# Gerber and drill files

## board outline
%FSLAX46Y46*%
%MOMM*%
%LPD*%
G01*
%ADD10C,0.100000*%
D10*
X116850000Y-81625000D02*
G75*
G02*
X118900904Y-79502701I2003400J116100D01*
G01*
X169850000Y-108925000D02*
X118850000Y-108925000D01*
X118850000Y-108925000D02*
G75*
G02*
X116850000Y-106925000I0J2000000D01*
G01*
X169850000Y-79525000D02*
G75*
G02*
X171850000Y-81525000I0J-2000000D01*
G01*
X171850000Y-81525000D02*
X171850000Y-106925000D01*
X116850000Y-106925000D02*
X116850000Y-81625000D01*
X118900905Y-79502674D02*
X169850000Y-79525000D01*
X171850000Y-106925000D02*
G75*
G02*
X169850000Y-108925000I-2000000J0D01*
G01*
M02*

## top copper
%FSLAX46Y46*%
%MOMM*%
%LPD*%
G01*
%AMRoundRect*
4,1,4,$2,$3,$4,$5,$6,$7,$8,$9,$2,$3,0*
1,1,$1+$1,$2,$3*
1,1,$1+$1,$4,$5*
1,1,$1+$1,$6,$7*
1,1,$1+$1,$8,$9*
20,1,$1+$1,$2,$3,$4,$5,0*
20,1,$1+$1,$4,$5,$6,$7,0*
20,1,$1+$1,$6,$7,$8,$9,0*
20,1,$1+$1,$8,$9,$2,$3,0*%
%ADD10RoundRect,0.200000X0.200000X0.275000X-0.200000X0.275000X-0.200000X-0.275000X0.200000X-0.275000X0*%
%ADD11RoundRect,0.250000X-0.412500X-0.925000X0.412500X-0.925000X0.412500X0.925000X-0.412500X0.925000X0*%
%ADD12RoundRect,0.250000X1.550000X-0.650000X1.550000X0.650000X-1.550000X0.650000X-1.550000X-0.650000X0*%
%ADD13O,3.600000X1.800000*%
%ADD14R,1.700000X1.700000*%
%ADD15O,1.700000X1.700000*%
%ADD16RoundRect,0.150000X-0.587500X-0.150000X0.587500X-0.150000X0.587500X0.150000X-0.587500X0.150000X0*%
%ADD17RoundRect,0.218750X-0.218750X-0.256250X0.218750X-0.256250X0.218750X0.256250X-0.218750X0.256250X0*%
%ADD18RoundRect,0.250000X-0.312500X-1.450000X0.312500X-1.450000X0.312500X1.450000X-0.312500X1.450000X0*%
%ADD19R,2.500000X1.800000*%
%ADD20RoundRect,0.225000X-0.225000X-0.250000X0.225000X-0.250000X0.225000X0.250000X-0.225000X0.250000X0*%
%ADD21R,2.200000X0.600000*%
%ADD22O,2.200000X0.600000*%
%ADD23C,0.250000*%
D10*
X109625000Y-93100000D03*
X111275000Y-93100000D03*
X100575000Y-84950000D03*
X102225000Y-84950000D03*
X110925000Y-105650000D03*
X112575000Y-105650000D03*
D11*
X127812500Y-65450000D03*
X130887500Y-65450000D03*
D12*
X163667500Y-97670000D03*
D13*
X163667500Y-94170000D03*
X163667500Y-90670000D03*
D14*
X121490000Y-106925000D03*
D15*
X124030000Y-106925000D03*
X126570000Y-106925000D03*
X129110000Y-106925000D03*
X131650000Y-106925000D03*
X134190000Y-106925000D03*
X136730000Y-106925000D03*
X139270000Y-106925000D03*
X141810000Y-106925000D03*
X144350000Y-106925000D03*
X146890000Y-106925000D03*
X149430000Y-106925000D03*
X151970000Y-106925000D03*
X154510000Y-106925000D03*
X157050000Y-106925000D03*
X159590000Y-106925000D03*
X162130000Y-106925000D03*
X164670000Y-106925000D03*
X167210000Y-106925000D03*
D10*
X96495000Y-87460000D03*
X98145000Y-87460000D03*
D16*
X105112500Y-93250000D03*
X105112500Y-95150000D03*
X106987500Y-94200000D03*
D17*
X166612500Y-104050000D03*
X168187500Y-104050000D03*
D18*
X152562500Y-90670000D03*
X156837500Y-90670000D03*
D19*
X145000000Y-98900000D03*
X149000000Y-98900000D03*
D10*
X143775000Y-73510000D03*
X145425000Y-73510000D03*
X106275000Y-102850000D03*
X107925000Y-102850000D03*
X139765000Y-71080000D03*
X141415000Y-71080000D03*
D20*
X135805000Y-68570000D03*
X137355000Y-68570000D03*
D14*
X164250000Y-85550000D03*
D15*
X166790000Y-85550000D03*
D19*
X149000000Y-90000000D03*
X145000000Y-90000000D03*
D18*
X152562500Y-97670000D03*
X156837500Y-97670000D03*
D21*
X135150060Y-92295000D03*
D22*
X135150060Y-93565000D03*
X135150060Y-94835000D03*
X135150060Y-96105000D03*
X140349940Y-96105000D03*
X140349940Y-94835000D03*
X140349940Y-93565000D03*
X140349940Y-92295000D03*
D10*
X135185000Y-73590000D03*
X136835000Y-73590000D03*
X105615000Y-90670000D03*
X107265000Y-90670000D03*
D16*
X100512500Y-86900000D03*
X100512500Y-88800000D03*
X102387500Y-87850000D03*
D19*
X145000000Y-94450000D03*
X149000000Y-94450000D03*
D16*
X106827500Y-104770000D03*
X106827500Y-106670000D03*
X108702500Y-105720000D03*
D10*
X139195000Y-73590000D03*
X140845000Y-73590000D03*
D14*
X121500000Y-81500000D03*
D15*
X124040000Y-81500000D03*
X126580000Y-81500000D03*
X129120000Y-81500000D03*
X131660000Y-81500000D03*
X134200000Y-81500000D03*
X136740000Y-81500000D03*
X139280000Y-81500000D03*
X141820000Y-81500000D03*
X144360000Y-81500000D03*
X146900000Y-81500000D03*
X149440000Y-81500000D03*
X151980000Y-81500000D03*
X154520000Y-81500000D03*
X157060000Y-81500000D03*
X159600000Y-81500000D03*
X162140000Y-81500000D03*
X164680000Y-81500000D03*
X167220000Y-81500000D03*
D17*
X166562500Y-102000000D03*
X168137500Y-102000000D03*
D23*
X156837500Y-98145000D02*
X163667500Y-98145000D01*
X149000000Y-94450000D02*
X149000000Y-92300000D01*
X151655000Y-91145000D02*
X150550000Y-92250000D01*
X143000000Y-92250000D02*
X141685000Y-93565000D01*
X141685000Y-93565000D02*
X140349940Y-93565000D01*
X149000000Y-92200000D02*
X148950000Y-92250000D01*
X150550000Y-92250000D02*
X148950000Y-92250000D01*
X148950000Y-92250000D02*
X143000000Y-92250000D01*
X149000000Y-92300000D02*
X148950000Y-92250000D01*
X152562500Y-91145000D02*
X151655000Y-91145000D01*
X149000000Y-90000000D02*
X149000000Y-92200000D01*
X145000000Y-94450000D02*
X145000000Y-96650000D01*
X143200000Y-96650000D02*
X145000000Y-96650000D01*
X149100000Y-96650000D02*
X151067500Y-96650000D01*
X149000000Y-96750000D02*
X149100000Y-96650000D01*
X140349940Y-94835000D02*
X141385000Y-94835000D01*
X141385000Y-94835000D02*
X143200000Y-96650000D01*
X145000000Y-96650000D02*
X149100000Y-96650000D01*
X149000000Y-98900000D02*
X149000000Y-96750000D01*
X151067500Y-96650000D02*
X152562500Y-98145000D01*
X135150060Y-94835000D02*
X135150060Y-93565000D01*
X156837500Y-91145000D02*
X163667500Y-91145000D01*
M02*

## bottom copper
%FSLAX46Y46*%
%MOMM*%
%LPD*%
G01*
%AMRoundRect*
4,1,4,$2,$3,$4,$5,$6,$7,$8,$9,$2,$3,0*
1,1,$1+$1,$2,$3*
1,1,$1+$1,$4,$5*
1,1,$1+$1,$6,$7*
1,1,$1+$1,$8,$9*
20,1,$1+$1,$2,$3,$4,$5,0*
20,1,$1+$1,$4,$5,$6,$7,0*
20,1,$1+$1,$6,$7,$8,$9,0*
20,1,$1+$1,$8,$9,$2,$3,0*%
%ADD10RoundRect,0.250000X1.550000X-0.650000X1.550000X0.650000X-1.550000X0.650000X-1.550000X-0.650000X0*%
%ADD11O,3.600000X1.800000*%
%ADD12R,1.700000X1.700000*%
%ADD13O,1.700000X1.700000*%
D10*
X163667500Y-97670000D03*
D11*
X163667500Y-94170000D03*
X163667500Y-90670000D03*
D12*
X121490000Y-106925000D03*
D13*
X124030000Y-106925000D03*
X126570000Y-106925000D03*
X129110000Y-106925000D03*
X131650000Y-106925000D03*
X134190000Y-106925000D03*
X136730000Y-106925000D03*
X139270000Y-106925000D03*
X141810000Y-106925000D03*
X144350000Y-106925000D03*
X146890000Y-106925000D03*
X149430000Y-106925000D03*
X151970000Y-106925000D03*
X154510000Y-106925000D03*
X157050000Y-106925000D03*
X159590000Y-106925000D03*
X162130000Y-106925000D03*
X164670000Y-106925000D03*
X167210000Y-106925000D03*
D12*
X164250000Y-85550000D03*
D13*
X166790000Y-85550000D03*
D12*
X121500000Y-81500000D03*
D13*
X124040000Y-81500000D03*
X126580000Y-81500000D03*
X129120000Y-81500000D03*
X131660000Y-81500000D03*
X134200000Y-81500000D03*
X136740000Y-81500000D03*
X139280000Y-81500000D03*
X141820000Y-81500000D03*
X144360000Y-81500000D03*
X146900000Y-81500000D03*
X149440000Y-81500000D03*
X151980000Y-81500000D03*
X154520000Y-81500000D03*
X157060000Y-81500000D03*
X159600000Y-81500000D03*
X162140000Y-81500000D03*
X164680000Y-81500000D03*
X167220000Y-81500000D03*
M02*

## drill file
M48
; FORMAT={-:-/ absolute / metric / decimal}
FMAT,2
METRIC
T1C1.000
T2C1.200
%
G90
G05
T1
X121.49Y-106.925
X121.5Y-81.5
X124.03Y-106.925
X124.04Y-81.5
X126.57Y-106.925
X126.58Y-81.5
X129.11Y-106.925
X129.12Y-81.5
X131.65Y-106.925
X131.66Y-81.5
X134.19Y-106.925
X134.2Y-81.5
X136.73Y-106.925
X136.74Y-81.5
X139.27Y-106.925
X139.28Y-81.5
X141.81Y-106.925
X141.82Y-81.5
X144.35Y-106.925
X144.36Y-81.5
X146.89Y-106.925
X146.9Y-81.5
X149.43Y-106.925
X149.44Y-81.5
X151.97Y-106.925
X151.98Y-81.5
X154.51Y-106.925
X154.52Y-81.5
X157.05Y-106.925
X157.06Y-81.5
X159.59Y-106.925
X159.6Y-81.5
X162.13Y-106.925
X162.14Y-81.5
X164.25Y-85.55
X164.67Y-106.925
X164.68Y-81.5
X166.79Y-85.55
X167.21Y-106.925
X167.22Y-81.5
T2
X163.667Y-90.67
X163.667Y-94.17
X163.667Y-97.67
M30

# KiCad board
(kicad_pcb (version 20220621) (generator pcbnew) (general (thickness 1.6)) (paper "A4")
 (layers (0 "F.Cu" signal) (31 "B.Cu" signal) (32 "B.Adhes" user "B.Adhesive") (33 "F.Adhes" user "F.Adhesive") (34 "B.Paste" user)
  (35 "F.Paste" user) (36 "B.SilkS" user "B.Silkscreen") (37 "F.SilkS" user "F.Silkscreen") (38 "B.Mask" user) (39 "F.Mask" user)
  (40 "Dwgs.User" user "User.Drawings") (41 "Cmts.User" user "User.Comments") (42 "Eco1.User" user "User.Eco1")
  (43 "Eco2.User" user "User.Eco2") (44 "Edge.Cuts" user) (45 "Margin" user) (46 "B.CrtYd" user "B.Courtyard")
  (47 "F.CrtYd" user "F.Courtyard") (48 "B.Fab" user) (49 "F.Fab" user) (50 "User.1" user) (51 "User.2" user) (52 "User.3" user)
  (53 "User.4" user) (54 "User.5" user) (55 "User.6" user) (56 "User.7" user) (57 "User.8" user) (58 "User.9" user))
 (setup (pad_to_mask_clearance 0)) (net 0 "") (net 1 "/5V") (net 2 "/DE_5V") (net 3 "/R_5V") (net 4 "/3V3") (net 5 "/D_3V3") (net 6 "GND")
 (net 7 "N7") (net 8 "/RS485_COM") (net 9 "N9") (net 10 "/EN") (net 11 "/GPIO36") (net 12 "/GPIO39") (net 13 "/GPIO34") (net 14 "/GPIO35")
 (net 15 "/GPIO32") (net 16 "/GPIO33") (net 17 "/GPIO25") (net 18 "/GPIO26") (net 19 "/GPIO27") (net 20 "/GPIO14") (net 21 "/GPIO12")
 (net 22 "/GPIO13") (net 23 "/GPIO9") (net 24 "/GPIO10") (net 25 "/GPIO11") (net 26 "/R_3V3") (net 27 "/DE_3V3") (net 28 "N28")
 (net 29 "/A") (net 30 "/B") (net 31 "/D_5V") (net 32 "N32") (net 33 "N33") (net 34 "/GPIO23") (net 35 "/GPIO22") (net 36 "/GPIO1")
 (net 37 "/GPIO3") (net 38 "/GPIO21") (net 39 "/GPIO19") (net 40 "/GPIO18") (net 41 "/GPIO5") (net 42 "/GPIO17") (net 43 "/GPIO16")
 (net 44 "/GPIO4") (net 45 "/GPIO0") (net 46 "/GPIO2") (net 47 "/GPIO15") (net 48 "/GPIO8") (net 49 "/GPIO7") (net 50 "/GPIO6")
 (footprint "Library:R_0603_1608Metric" (layer "F.Cu") (at 110.45 93.1)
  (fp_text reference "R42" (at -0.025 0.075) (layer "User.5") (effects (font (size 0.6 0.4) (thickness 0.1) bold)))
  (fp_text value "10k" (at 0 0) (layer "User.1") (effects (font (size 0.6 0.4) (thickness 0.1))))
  (pad "1" smd roundrect (at -0.825 0 180) (size 0.8 0.95) (layers "F.Cu" "F.Paste" "F.Mask") (roundrect_rratio 0.25) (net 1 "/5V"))
  (pad "2" smd roundrect (at 0.825 0 180) (size 0.8 0.95) (layers "F.Cu" "F.Paste" "F.Mask") (roundrect_rratio 0.25) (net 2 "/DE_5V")))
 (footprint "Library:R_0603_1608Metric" (layer "F.Cu") (at 101.4 84.95)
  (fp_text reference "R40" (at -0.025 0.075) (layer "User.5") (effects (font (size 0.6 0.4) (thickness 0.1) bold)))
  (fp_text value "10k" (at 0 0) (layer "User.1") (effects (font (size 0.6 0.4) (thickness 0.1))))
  (pad "1" smd roundrect (at -0.825 0 180) (size 0.8 0.95) (layers "F.Cu" "F.Paste" "F.Mask") (roundrect_rratio 0.25) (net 1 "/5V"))
  (pad "2" smd roundrect (at 0.825 0 180) (size 0.8 0.95) (layers "F.Cu" "F.Paste" "F.Mask") (roundrect_rratio 0.25) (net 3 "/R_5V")))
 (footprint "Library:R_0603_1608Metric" (layer "F.Cu") (at 111.75 105.65)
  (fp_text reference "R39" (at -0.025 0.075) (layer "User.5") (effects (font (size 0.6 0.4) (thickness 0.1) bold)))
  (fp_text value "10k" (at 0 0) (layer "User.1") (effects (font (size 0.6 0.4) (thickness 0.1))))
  (pad "1" smd roundrect (at -0.825 0 180) (size 0.8 0.95) (layers "F.Cu" "F.Paste" "F.Mask") (roundrect_rratio 0.25) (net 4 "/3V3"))
  (pad "2" smd roundrect (at 0.825 0 180) (size 0.8 0.95) (layers "F.Cu" "F.Paste" "F.Mask") (roundrect_rratio 0.25) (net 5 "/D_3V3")))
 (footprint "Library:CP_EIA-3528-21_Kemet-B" (layer "F.Cu") (at 129.35 65.45)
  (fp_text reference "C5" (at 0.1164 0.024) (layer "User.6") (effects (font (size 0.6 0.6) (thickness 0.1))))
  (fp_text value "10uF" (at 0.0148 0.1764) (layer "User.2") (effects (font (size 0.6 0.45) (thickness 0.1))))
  (pad "1" smd roundrect (at -1.5375 0) (size 1.325 2.35) (layers "F.Cu" "F.Paste" "F.Mask") (roundrect_rratio 0.1886792453) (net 1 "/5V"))
  (pad "2" smd roundrect (at 1.5375 0) (size 1.325 2.35) (layers "F.Cu" "F.Paste" "F.Mask") (roundrect_rratio 0.1886792453) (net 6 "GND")))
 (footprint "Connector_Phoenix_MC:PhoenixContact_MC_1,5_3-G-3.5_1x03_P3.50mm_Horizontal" (layer "F.Cu") (at 163.6675 97.67 90)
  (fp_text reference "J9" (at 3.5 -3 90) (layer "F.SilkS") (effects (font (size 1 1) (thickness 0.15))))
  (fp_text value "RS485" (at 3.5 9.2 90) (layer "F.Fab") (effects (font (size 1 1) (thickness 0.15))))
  (pad "1" thru_hole roundrect (at 0 0 90) (size 1.8 3.6) (drill 1.2) (layers *.Cu *.Mask) (roundrect_rratio 0.138889) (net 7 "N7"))
  (pad "2" thru_hole oval (at 3.5 0 90) (size 1.8 3.6) (drill 1.2) (layers *.Cu *.Mask) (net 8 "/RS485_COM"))
  (pad "3" thru_hole oval (at 7 0 90) (size 1.8 3.6) (drill 1.2) (layers *.Cu *.Mask) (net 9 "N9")))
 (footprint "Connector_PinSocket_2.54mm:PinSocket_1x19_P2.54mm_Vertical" (layer "F.Cu") (at 121.49 106.925 90)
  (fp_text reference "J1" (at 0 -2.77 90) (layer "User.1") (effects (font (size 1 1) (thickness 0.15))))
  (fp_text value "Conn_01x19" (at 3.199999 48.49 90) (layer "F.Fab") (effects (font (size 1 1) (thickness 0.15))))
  (pad "1" thru_hole rect (at 0 0 90) (size 1.7 1.7) (drill 1) (layers *.Cu *.Mask) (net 4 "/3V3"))
  (pad "2" thru_hole oval (at 0 2.54 90) (size 1.7 1.7) (drill 1) (layers *.Cu *.Mask) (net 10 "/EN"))
  (pad "3" thru_hole oval (at 0 5.08 90) (size 1.7 1.7) (drill 1) (layers *.Cu *.Mask) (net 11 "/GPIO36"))
  (pad "4" thru_hole oval (at 0 7.62 90) (size 1.7 1.7) (drill 1) (layers *.Cu *.Mask) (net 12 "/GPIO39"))
  (pad "5" thru_hole oval (at 0 10.16 90) (size 1.7 1.7) (drill 1) (layers *.Cu *.Mask) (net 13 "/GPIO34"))
  (pad "6" thru_hole oval (at 0 12.7 90) (size 1.7 1.7) (drill 1) (layers *.Cu *.Mask) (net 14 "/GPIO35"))
  (pad "7" thru_hole oval (at 0 15.24 90) (size 1.7 1.7) (drill 1) (layers *.Cu *.Mask) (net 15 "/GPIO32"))
  (pad "8" thru_hole oval (at 0 17.78 90) (size 1.7 1.7) (drill 1) (layers *.Cu *.Mask) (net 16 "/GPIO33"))
  (pad "9" thru_hole oval (at 0 20.32 90) (size 1.7 1.7) (drill 1) (layers *.Cu *.Mask) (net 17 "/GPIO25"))
  (pad "10" thru_hole oval (at 0 22.86 90) (size 1.7 1.7) (drill 1) (layers *.Cu *.Mask) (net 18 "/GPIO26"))
  (pad "11" thru_hole oval (at 0 25.4 90) (size 1.7 1.7) (drill 1) (layers *.Cu *.Mask) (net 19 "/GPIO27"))
  (pad "12" thru_hole oval (at 0 27.94 90) (size 1.7 1.7) (drill 1) (layers *.Cu *.Mask) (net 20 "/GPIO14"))
  (pad "13" thru_hole oval (at 0 30.48 90) (size 1.7 1.7) (drill 1) (layers *.Cu *.Mask) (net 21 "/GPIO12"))
  (pad "14" thru_hole oval (at 0 33.02 90) (size 1.7 1.7) (drill 1) (layers *.Cu *.Mask) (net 6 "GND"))
  (pad "15" thru_hole oval (at 0 35.56 90) (size 1.7 1.7) (drill 1) (layers *.Cu *.Mask) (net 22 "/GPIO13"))
  (pad "16" thru_hole oval (at 0 38.1 90) (size 1.7 1.7) (drill 1) (layers *.Cu *.Mask) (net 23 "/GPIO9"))
  (pad "17" thru_hole oval (at 0 40.64 90) (size 1.7 1.7) (drill 1) (layers *.Cu *.Mask) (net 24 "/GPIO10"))
  (pad "18" thru_hole oval (at 0 43.18 90) (size 1.7 1.7) (drill 1) (layers *.Cu *.Mask) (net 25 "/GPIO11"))
  (pad "19" thru_hole oval (at 0 45.72 90) (size 1.7 1.7) (drill 1) (layers *.Cu *.Mask) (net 1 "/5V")))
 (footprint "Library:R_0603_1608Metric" (layer "F.Cu") (at 97.32 87.46)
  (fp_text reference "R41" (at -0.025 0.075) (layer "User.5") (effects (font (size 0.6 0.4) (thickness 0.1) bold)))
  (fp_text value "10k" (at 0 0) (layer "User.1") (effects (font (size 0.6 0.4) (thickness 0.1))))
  (pad "1" smd roundrect (at -0.825 0 180) (size 0.8 0.95) (layers "F.Cu" "F.Paste" "F.Mask") (roundrect_rratio 0.25) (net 4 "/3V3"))
  (pad "2" smd roundrect (at 0.825 0 180) (size 0.8 0.95) (layers "F.Cu" "F.Paste" "F.Mask") (roundrect_rratio 0.25) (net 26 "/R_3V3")))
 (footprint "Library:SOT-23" (layer "F.Cu") (at 106.05 94.2)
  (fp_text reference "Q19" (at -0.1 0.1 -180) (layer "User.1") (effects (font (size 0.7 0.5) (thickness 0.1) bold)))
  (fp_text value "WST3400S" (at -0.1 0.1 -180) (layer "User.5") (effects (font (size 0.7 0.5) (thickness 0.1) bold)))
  (pad "1" smd roundrect (at -0.9375 -0.95) (size 1.475 0.6) (layers "F.Cu" "F.Paste" "F.Mask") (roundrect_rratio 0.25) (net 4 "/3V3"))
  (pad "2" smd roundrect (at -0.9375 0.95) (size 1.475 0.6) (layers "F.Cu" "F.Paste" "F.Mask") (roundrect_rratio 0.25) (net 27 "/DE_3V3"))
  (pad "3" smd roundrect (at 0.9375 0) (size 1.475 0.6) (layers "F.Cu" "F.Paste" "F.Mask") (roundrect_rratio 0.25) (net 2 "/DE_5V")))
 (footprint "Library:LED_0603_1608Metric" (layer "F.Cu") (at 167.4 104.05)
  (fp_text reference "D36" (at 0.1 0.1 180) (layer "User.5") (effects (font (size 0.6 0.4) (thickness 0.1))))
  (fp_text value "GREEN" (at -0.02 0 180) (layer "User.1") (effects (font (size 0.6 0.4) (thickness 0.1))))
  (pad "1" smd roundrect (at -0.7875 0) (size 0.875 0.95) (layers "F.Cu" "F.Paste" "F.Mask") (roundrect_rratio 0.25) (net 6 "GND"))
  (pad "2" smd roundrect (at 0.7875 0) (size 0.875 0.95) (layers "F.Cu" "F.Paste" "F.Mask") (roundrect_rratio 0.25) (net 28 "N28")))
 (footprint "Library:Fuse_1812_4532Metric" (layer "F.Cu") (at 154.7 90.67)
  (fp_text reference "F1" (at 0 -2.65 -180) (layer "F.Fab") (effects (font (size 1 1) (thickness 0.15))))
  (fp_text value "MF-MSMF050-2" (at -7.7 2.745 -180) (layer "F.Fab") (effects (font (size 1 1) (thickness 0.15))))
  (pad "1" smd roundrect (at -2.1375 0) (size 1.125 3.4) (layers "F.Cu" "F.Paste" "F.Mask") (roundrect_rratio 0.2222222222) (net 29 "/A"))
  (pad "2" smd roundrect (at 2.1375 0) (size 1.125 3.4) (layers "F.Cu" "F.Paste" "F.Mask") (roundrect_rratio 0.2222222222) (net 9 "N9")))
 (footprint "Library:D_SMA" (layer "F.Cu") (at 147 98.9)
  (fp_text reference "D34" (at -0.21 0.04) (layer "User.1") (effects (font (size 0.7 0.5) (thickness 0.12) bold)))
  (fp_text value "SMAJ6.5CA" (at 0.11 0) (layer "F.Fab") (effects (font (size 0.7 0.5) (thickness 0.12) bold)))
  (pad "1" smd rect (at -2 0) (size 2.5 1.8) (layers "F.Cu" "F.Paste" "F.Mask") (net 8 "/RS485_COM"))
  (pad "2" smd rect (at 2 0) (size 2.5 1.8) (layers "F.Cu" "F.Paste" "F.Mask") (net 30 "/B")))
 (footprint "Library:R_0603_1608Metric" (layer "F.Cu") (at 144.6 73.51)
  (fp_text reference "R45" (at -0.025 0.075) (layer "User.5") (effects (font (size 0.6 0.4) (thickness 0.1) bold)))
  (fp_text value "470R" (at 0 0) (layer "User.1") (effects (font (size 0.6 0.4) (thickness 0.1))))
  (pad "1" smd roundrect (at -0.825 0 180) (size 0.8 0.95) (layers "F.Cu" "F.Paste" "F.Mask") (roundrect_rratio 0.25) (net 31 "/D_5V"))
  (pad "2" smd roundrect (at 0.825 0 180) (size 0.8 0.95) (layers "F.Cu" "F.Paste" "F.Mask") (roundrect_rratio 0.25) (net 28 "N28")))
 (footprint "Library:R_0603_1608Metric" (layer "F.Cu") (at 107.1 102.85)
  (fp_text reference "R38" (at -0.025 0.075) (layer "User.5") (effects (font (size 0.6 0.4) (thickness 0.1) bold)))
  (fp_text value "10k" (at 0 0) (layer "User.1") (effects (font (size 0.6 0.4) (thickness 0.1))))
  (pad "1" smd roundrect (at -0.825 0 180) (size 0.8 0.95) (layers "F.Cu" "F.Paste" "F.Mask") (roundrect_rratio 0.25) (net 1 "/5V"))
  (pad "2" smd roundrect (at 0.825 0 180) (size 0.8 0.95) (layers "F.Cu" "F.Paste" "F.Mask") (roundrect_rratio 0.25) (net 31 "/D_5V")))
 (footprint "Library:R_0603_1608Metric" (layer "F.Cu") (at 140.59 71.08)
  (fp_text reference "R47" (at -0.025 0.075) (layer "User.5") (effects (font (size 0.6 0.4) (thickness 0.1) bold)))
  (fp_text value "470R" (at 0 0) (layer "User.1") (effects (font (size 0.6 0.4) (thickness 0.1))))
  (pad "1" smd roundrect (at -0.825 0 180) (size 0.8 0.95) (layers "F.Cu" "F.Paste" "F.Mask") (roundrect_rratio 0.25) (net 3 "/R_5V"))
  (pad "2" smd roundrect (at 0.825 0 180) (size 0.8 0.95) (layers "F.Cu" "F.Paste" "F.Mask") (roundrect_rratio 0.25) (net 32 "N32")))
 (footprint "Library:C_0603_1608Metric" (layer "F.Cu") (at 136.58 68.57)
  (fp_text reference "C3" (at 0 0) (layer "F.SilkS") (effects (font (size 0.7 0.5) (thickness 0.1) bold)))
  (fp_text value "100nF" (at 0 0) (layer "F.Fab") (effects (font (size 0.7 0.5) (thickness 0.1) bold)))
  (pad "1" smd roundrect (at -0.775 0) (size 0.9 0.95) (layers "F.Cu" "F.Paste" "F.Mask") (roundrect_rratio 0.25) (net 1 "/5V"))
  (pad "2" smd roundrect (at 0.775 0) (size 0.9 0.95) (layers "F.Cu" "F.Paste" "F.Mask") (roundrect_rratio 0.25) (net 6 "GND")))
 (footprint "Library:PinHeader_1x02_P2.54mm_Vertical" (layer "F.Cu") (at 164.25 85.55 90)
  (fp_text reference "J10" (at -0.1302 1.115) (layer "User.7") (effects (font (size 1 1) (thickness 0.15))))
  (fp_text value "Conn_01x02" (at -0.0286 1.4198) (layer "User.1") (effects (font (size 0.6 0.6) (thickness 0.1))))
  (pad "1" thru_hole rect locked (at 0 0 90) (size 1.7 1.7) (drill 1) (layers *.Cu *.Mask) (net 7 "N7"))
  (pad "2" thru_hole oval locked (at 0 2.54 90) (size 1.7 1.7) (drill 1) (layers *.Cu *.Mask) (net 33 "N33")))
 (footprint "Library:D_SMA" (layer "F.Cu") (at 147 90 180)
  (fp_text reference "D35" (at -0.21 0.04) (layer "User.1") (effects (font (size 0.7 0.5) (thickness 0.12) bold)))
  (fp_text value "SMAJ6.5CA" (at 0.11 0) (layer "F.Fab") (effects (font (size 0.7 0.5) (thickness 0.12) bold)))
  (pad "1" smd rect (at -2 0 180) (size 2.5 1.8) (layers "F.Cu" "F.Paste" "F.Mask") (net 29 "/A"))
  (pad "2" smd rect (at 2 0 180) (size 2.5 1.8) (layers "F.Cu" "F.Paste" "F.Mask") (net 8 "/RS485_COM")))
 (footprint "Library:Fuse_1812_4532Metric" (layer "F.Cu") (at 154.7 97.67)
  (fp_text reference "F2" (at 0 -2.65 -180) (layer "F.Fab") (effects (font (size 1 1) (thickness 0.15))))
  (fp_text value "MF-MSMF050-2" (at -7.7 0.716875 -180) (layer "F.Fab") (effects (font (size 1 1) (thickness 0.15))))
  (pad "1" smd roundrect (at -2.1375 0) (size 1.125 3.4) (layers "F.Cu" "F.Paste" "F.Mask") (roundrect_rratio 0.2222222222) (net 30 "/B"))
  (pad "2" smd roundrect (at 2.1375 0) (size 1.125 3.4) (layers "F.Cu" "F.Paste" "F.Mask") (roundrect_rratio 0.2222222222) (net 7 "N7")))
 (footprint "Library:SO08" (layer "F.Cu") (at 137.75 94.2 -90)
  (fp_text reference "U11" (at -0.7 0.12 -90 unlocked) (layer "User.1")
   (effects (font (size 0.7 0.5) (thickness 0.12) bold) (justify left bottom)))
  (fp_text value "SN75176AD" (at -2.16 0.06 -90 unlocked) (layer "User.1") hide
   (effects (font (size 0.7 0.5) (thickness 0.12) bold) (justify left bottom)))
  (pad "1" smd rect (at -1.905 2.59994 270) (size 0.6 2.2) (layers "F.Cu" "F.Paste" "F.Mask") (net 3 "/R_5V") (thermal_bridge_angle 45))
  (pad "2" smd oval (at -0.635 2.59994 270) (size 0.6 2.2) (layers "F.Cu" "F.Paste" "F.Mask") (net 2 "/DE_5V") (thermal_bridge_angle 45))
  (pad "3" smd oval (at 0.635 2.59994 270) (size 0.6 2.2) (layers "F.Cu" "F.Paste" "F.Mask") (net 2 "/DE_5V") (thermal_bridge_angle 45))
  (pad "4" smd oval (at 1.905 2.59994 270) (size 0.6 2.2) (layers "F.Cu" "F.Paste" "F.Mask") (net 31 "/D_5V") (thermal_bridge_angle 45))
  (pad "5" smd oval (at 1.905 -2.59994 270) (size 0.6 2.2) (layers "F.Cu" "F.Paste" "F.Mask") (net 6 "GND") (thermal_bridge_angle 45))
  (pad "6" smd oval (at 0.635 -2.59994 270) (size 0.6 2.2) (layers "F.Cu" "F.Paste" "F.Mask") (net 30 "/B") (thermal_bridge_angle 45))
  (pad "7" smd oval (at -0.635 -2.59994 270) (size 0.6 2.2) (layers "F.Cu" "F.Paste" "F.Mask") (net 29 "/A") (thermal_bridge_angle 45))
  (pad "8" smd oval (at -1.905 -2.59994 90) (size 0.6 2.2) (layers "F.Cu" "F.Paste" "F.Mask") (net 1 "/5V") (thermal_bridge_angle 45)))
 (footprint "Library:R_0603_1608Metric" (layer "F.Cu") (at 136.01 73.59)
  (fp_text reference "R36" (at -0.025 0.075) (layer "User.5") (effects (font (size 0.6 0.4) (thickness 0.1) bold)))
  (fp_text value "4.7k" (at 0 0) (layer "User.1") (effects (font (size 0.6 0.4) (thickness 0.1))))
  (pad "1" smd roundrect (at -0.825 0 180) (size 0.8 0.95) (layers "F.Cu" "F.Paste" "F.Mask") (roundrect_rratio 0.25) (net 9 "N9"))
  (pad "2" smd roundrect (at 0.825 0 180) (size 0.8 0.95) (layers "F.Cu" "F.Paste" "F.Mask") (roundrect_rratio 0.25) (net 33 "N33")))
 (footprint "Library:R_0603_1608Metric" (layer "F.Cu") (at 106.44 90.67)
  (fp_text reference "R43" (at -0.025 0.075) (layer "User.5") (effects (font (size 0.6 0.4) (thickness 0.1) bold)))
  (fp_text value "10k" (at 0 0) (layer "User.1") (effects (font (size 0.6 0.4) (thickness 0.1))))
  (pad "1" smd roundrect (at -0.825 0 180) (size 0.8 0.95) (layers "F.Cu" "F.Paste" "F.Mask") (roundrect_rratio 0.25) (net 4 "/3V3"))
  (pad "2" smd roundrect (at 0.825 0 180) (size 0.8 0.95) (layers "F.Cu" "F.Paste" "F.Mask") (roundrect_rratio 0.25) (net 27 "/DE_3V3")))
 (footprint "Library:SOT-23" (layer "F.Cu") (at 101.45 87.85)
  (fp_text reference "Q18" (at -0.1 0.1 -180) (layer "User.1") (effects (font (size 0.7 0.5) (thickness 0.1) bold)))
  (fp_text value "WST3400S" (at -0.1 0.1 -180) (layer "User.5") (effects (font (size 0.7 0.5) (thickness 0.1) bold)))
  (pad "1" smd roundrect (at -0.9375 -0.95) (size 1.475 0.6) (layers "F.Cu" "F.Paste" "F.Mask") (roundrect_rratio 0.25) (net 4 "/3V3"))
  (pad "2" smd roundrect (at -0.9375 0.95) (size 1.475 0.6) (layers "F.Cu" "F.Paste" "F.Mask") (roundrect_rratio 0.25) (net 26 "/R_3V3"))
  (pad "3" smd roundrect (at 0.9375 0) (size 1.475 0.6) (layers "F.Cu" "F.Paste" "F.Mask") (roundrect_rratio 0.25) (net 3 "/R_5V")))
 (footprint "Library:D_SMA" (layer "F.Cu") (at 147 94.45)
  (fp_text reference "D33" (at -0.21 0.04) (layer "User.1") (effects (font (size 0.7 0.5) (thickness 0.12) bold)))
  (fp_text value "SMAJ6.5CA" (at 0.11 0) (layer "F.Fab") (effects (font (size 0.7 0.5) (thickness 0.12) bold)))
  (pad "1" smd rect (at -2 0) (size 2.5 1.8) (layers "F.Cu" "F.Paste" "F.Mask") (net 30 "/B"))
  (pad "2" smd rect (at 2 0) (size 2.5 1.8) (layers "F.Cu" "F.Paste" "F.Mask") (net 29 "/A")))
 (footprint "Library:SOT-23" (layer "F.Cu") (at 107.765 105.72)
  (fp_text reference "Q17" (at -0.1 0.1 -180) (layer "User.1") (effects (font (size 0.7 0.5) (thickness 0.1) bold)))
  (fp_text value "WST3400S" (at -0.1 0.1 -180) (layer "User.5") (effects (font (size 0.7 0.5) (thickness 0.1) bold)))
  (pad "1" smd roundrect (at -0.9375 -0.95) (size 1.475 0.6) (layers "F.Cu" "F.Paste" "F.Mask") (roundrect_rratio 0.25) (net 4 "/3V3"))
  (pad "2" smd roundrect (at -0.9375 0.95) (size 1.475 0.6) (layers "F.Cu" "F.Paste" "F.Mask") (roundrect_rratio 0.25) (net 5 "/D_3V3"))
  (pad "3" smd roundrect (at 0.9375 0) (size 1.475 0.6) (layers "F.Cu" "F.Paste" "F.Mask") (roundrect_rratio 0.25) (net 31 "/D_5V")))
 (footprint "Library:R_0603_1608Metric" (layer "F.Cu") (at 140.02 73.59)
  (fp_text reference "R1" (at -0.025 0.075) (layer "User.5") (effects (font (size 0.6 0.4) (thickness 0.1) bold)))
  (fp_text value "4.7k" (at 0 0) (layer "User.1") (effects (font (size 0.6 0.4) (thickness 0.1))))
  (pad "1" smd roundrect (at -0.825 0 180) (size 0.8 0.95) (layers "F.Cu" "F.Paste" "F.Mask") (roundrect_rratio 0.25) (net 3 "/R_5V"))
  (pad "2" smd roundrect (at 0.825 0 180) (size 0.8 0.95) (layers "F.Cu" "F.Paste" "F.Mask") (roundrect_rratio 0.25) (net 1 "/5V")))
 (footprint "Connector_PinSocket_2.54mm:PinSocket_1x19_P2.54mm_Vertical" (layer "F.Cu") (at 121.5 81.5 90)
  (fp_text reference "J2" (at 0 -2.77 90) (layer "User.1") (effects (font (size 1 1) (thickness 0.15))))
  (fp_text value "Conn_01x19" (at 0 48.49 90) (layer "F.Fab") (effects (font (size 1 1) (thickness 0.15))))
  (pad "1" thru_hole rect (at 0 0 90) (size 1.7 1.7) (drill 1) (layers *.Cu *.Mask) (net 6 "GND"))
  (pad "2" thru_hole oval (at 0 2.54 90) (size 1.7 1.7) (drill 1) (layers *.Cu *.Mask) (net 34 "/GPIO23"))
  (pad "3" thru_hole oval (at 0 5.08 90) (size 1.7 1.7) (drill 1) (layers *.Cu *.Mask) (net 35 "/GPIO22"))
  (pad "4" thru_hole oval (at 0 7.62 90) (size 1.7 1.7) (drill 1) (layers *.Cu *.Mask) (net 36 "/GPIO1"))
  (pad "5" thru_hole oval (at 0 10.16 90) (size 1.7 1.7) (drill 1) (layers *.Cu *.Mask) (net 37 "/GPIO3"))
  (pad "6" thru_hole oval (at 0 12.7 90) (size 1.7 1.7) (drill 1) (layers *.Cu *.Mask) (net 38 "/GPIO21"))
  (pad "7" thru_hole oval (at 0 15.24 90) (size 1.7 1.7) (drill 1) (layers *.Cu *.Mask) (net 6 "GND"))
  (pad "8" thru_hole oval (at 0 17.78 90) (size 1.7 1.7) (drill 1) (layers *.Cu *.Mask) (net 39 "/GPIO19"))
  (pad "9" thru_hole oval (at 0 20.32 90) (size 1.7 1.7) (drill 1) (layers *.Cu *.Mask) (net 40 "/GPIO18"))
  (pad "10" thru_hole oval (at 0 22.86 90) (size 1.7 1.7) (drill 1) (layers *.Cu *.Mask) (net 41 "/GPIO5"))
  (pad "11" thru_hole oval (at 0 25.4 90) (size 1.7 1.7) (drill 1) (layers *.Cu *.Mask) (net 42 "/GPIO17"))
  (pad "12" thru_hole oval (at 0 27.94 90) (size 1.7 1.7) (drill 1) (layers *.Cu *.Mask) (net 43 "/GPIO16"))
  (pad "13" thru_hole oval (at 0 30.48 90) (size 1.7 1.7) (drill 1) (layers *.Cu *.Mask) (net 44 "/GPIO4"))
  (pad "14" thru_hole oval (at 0 33.02 90) (size 1.7 1.7) (drill 1) (layers *.Cu *.Mask) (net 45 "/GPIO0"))
  (pad "15" thru_hole oval (at 0 35.56 90) (size 1.7 1.7) (drill 1) (layers *.Cu *.Mask) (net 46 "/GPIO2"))
  (pad "16" thru_hole oval (at 0 38.1 90) (size 1.7 1.7) (drill 1) (layers *.Cu *.Mask) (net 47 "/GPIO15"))
  (pad "17" thru_hole oval (at 0 40.64 90) (size 1.7 1.7) (drill 1) (layers *.Cu *.Mask) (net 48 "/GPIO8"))
  (pad "18" thru_hole oval (at 0 43.18 90) (size 1.7 1.7) (drill 1) (layers *.Cu *.Mask) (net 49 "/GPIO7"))
  (pad "19" thru_hole oval (at 0 45.72 90) (size 1.7 1.7) (drill 1) (layers *.Cu *.Mask) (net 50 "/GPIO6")))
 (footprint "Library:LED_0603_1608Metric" (layer "F.Cu") (at 167.35 102)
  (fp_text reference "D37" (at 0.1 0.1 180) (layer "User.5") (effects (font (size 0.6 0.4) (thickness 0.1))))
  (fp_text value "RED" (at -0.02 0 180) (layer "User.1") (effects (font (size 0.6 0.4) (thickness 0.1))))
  (pad "1" smd roundrect (at -0.7875 0) (size 0.875 0.95) (layers "F.Cu" "F.Paste" "F.Mask") (roundrect_rratio 0.25) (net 6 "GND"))
  (pad "2" smd roundrect (at 0.7875 0) (size 0.875 0.95) (layers "F.Cu" "F.Paste" "F.Mask") (roundrect_rratio 0.25) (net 32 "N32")))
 (gr_arc (start 116.85 81.625) (mid 117.410345 80.114382) (end 118.900905 79.502674) (stroke (width 0.1) (type default)) (layer "Edge.Cuts"))
 (gr_line (start 169.85 108.925) (end 118.85 108.925) (stroke (width 0.1) (type default)) (layer "Edge.Cuts"))
 (gr_arc (start 118.85 108.925) (mid 117.435786 108.339214) (end 116.85 106.925) (stroke (width 0.1) (type default)) (layer "Edge.Cuts"))
 (gr_arc (start 169.85 79.525) (mid 171.264214 80.110786) (end 171.85 81.525) (stroke (width 0.1) (type default)) (layer "Edge.Cuts"))
 (gr_line (start 171.85 81.525) (end 171.85 106.925) (stroke (width 0.1) (type default)) (layer "Edge.Cuts"))
 (gr_line (start 116.85 106.925) (end 116.85 81.625) (stroke (width 0.1) (type default)) (layer "Edge.Cuts"))
 (gr_line (start 118.900905 79.502674) (end 169.85 79.525) (stroke (width 0.1) (type default)) (layer "Edge.Cuts"))
 (gr_arc (start 171.85 106.925) (mid 171.264214 108.339214) (end 169.85 108.925) (stroke (width 0.1) (type default)) (layer "Edge.Cuts"))
 (segment (start 156.8375 98.145) (end 163.6675 98.145) (width 0.25) (layer "F.Cu") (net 7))
 (segment (start 149 94.45) (end 149 92.3) (width 0.25) (layer "F.Cu") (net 29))
 (segment (start 151.655 91.145) (end 150.55 92.25) (width 0.25) (layer "F.Cu") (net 29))
 (segment (start 143 92.25) (end 141.685 93.565) (width 0.25) (layer "F.Cu") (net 29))
 (segment (start 141.685 93.565) (end 140.34994 93.565) (width 0.25) (layer "F.Cu") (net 29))
 (segment (start 149 92.2) (end 148.95 92.25) (width 0.25) (layer "F.Cu") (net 29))
 (segment (start 150.55 92.25) (end 148.95 92.25) (width 0.25) (layer "F.Cu") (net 29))
 (segment (start 148.95 92.25) (end 143 92.25) (width 0.25) (layer "F.Cu") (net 29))
 (segment (start 149 92.3) (end 148.95 92.25) (width 0.25) (layer "F.Cu") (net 29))
 (segment (start 152.5625 91.145) (end 151.655 91.145) (width 0.25) (layer "F.Cu") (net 29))
 (segment (start 149 90) (end 149 92.2) (width 0.25) (layer "F.Cu") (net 29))
 (segment (start 145 94.45) (end 145 96.65) (width 0.25) (layer "F.Cu") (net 30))
 (segment (start 143.2 96.65) (end 145 96.65) (width 0.25) (layer "F.Cu") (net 30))
 (segment (start 149.1 96.65) (end 151.0675 96.65) (width 0.25) (layer "F.Cu") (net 30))
 (segment (start 149 96.75) (end 149.1 96.65) (width 0.25) (layer "F.Cu") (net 30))
 (segment (start 140.34994 94.835) (end 141.385 94.835) (width 0.25) (layer "F.Cu") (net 30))
 (segment (start 141.385 94.835) (end 143.2 96.65) (width 0.25) (layer "F.Cu") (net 30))
 (segment (start 145 96.65) (end 149.1 96.65) (width 0.25) (layer "F.Cu") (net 30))
 (segment (start 149 98.9) (end 149 96.75) (width 0.25) (layer "F.Cu") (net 30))
 (segment (start 151.0675 96.65) (end 152.5625 98.145) (width 0.25) (layer "F.Cu") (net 30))
 (segment (start 135.15006 94.835) (end 135.15006 93.565) (width 0.25) (layer "F.Cu") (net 2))
 (segment (start 156.8375 91.145) (end 163.6675 91.145) (width 0.25) (layer "F.Cu") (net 9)))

